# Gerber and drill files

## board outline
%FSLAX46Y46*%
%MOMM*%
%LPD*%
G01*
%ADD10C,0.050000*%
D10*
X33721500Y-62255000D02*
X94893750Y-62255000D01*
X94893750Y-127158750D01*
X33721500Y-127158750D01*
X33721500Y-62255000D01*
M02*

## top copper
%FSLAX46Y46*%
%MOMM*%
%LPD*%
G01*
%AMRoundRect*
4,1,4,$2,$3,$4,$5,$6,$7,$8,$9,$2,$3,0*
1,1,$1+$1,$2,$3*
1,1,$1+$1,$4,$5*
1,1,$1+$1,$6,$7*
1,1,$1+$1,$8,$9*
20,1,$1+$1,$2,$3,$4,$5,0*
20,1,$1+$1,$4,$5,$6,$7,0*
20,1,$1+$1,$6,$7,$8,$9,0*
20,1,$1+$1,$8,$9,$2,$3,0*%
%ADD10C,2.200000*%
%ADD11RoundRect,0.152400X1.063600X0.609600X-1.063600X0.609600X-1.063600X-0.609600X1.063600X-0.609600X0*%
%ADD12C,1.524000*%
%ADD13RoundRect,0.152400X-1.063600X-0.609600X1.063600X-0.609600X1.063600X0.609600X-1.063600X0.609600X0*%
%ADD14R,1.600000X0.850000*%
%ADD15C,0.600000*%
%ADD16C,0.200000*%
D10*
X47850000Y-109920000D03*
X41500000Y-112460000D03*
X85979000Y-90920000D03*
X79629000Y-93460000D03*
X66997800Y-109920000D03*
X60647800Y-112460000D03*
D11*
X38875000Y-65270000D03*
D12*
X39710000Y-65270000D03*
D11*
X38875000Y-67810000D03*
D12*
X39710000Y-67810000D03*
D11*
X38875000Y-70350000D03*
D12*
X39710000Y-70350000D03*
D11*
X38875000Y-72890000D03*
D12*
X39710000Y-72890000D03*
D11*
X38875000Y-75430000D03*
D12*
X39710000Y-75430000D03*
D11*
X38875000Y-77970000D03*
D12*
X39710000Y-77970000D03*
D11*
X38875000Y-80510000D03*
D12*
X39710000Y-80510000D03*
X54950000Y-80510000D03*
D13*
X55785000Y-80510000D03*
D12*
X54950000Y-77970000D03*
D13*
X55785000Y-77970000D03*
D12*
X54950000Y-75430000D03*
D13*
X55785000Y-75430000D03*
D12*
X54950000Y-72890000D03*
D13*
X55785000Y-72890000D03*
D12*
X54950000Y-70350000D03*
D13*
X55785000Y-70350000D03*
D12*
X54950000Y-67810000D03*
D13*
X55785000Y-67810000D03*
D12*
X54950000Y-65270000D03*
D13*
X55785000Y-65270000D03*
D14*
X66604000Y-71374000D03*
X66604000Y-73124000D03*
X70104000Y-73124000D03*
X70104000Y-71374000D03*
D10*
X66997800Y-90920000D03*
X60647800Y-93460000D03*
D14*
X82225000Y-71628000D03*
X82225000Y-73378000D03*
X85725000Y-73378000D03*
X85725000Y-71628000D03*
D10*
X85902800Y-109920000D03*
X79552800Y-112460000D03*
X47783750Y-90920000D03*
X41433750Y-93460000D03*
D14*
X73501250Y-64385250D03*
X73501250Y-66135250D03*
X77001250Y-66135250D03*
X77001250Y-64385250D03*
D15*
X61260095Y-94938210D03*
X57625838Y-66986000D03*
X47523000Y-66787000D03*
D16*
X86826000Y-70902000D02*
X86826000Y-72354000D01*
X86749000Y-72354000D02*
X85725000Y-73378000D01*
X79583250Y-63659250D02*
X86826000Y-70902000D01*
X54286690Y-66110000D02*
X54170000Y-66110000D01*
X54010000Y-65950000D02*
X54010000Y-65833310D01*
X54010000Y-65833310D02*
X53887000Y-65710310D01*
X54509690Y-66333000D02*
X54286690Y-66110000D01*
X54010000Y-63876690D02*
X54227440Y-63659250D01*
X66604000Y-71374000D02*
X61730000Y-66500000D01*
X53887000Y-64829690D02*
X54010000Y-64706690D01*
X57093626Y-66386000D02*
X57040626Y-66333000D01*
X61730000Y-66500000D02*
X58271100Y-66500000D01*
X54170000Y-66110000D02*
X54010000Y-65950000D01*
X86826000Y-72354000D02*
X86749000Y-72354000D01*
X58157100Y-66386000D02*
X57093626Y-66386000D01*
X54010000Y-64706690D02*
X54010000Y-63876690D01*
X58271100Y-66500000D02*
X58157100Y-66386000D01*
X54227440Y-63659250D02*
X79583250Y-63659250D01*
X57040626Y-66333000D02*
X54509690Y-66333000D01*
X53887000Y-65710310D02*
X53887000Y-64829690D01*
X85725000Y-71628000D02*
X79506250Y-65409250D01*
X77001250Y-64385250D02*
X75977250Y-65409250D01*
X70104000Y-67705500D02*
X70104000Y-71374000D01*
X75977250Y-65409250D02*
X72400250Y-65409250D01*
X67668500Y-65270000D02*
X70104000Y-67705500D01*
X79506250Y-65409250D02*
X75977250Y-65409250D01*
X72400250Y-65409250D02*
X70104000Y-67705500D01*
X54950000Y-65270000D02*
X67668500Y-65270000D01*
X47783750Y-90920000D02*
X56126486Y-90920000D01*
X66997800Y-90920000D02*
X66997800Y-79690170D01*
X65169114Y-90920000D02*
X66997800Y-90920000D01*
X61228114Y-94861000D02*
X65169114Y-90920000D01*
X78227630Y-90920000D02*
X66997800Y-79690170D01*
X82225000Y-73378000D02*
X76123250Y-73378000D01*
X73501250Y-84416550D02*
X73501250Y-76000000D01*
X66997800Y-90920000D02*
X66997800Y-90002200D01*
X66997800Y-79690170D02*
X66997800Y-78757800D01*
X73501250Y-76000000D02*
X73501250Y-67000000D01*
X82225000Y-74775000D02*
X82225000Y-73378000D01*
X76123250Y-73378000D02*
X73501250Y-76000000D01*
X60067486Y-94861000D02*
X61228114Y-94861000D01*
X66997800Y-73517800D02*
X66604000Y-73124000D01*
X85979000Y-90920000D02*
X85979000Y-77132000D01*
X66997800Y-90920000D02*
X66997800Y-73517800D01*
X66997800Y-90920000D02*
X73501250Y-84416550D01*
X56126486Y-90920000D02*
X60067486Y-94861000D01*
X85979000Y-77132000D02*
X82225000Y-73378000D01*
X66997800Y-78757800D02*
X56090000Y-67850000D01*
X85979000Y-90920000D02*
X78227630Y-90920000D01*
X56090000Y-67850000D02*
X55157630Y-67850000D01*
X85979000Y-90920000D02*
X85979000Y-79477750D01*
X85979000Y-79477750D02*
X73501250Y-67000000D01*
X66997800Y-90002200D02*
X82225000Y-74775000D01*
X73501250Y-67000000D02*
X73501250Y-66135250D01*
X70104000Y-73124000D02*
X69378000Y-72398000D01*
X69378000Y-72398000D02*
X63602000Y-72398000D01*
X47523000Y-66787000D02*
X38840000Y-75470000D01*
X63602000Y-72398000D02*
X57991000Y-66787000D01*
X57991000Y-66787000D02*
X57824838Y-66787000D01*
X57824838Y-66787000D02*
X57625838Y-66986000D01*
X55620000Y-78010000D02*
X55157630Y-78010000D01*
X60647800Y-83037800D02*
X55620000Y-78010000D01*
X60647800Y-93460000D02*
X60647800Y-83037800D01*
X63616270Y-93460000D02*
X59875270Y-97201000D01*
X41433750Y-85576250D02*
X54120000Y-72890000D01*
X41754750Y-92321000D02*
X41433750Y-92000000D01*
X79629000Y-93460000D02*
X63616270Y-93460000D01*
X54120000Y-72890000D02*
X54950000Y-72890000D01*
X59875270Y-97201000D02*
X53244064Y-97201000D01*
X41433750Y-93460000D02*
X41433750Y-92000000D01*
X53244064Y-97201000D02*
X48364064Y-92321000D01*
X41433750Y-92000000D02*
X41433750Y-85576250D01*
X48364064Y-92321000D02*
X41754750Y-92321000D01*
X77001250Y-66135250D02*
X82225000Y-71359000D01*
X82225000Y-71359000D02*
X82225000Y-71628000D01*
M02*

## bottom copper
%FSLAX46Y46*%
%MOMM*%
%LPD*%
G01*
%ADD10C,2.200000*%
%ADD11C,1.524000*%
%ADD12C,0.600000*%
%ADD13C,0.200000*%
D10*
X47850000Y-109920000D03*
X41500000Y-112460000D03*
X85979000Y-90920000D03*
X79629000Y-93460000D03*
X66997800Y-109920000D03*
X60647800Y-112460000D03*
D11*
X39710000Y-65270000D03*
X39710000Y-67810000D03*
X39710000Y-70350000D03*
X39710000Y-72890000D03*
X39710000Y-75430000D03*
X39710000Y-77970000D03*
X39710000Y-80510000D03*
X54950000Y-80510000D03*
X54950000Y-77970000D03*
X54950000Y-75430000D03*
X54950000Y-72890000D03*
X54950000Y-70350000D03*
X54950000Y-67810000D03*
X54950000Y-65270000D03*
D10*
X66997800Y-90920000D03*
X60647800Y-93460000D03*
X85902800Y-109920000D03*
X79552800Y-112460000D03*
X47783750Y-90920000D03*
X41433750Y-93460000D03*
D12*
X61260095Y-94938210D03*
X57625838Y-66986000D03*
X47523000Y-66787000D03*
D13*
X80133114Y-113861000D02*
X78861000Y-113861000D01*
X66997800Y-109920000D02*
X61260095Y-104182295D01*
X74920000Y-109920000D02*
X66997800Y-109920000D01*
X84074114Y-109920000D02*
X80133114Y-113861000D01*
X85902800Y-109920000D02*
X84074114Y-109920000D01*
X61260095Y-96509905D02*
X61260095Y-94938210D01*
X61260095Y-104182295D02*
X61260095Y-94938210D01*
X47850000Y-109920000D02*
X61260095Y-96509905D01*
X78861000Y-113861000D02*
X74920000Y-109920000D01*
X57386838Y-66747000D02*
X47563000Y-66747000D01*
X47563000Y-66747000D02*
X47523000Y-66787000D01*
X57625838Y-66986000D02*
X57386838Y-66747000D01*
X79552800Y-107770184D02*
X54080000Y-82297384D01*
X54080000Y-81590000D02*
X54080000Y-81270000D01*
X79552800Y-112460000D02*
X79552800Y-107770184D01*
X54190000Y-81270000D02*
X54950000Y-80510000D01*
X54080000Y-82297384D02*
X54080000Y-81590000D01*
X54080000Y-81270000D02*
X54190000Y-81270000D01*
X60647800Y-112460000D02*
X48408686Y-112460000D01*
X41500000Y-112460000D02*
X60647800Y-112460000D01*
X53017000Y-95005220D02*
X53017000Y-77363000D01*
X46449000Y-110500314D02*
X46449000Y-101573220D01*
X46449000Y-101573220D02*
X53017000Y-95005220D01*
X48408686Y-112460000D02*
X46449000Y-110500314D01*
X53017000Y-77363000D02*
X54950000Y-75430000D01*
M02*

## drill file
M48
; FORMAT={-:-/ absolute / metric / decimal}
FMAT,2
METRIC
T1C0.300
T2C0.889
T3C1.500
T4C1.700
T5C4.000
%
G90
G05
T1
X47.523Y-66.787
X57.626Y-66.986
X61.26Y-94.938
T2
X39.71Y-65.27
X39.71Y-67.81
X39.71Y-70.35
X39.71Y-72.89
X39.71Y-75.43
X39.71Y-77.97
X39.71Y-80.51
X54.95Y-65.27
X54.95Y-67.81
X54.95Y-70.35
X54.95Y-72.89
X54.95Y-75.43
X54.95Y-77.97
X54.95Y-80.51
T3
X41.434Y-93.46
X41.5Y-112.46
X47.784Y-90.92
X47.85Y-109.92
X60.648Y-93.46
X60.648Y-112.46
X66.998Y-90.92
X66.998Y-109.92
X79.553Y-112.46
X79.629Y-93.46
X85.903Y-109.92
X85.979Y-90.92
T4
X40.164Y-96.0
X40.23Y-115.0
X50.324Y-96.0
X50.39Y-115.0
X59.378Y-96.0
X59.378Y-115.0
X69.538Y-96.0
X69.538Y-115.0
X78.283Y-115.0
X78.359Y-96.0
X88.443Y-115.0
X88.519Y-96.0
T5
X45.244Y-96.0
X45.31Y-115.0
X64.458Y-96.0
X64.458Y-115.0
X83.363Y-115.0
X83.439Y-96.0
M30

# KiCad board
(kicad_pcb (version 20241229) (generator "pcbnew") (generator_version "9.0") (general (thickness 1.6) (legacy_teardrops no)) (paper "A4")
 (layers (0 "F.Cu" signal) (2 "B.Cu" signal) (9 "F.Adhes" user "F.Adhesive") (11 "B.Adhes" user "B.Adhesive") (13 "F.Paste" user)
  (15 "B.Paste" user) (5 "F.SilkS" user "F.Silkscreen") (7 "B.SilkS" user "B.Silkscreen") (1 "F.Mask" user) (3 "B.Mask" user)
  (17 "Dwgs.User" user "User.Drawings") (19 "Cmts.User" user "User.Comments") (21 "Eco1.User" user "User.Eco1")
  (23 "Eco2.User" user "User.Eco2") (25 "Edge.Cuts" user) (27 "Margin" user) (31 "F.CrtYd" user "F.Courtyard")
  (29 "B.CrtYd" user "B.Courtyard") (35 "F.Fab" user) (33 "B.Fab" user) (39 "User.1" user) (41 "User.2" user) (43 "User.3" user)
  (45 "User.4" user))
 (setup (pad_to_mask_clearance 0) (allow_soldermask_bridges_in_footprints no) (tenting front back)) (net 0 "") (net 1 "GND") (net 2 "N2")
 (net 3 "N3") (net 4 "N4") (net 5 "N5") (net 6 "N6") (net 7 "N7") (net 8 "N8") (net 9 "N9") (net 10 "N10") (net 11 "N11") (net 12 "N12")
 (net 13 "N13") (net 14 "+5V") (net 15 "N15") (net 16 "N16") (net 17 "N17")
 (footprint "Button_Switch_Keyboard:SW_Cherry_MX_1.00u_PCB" (layer "F.Cu") (at 47.85 109.92)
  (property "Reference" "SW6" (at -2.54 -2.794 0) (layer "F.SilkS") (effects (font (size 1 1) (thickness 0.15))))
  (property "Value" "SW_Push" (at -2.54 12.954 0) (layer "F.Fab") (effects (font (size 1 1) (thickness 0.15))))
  (pad "" np_thru_hole circle (at -7.62 5.08) (size 1.7 1.7) (drill 1.7) (layers "*.Cu" "*.Mask"))
  (pad "" np_thru_hole circle (at -2.54 5.08) (size 4 4) (drill 4) (layers "*.Cu" "*.Mask"))
  (pad "" np_thru_hole circle (at 2.54 5.08) (size 1.7 1.7) (drill 1.7) (layers "*.Cu" "*.Mask"))
  (pad "1" thru_hole circle (at 0 0) (size 2.2 2.2) (drill 1.5) (layers "*.Cu" "*.Mask") (remove_unused_layers no) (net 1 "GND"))
  (pad "2" thru_hole circle (at -6.35 2.54) (size 2.2 2.2) (drill 1.5) (layers "*.Cu" "*.Mask") (remove_unused_layers no) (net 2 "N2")))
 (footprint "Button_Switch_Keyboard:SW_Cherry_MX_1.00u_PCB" (layer "F.Cu") (at 85.979 90.92)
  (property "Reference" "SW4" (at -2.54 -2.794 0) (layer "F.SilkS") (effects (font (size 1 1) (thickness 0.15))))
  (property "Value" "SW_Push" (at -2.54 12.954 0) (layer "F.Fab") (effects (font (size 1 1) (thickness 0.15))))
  (pad "" np_thru_hole circle (at -7.62 5.08) (size 1.7 1.7) (drill 1.7) (layers "*.Cu" "*.Mask"))
  (pad "" np_thru_hole circle (at -2.54 5.08) (size 4 4) (drill 4) (layers "*.Cu" "*.Mask"))
  (pad "" np_thru_hole circle (at 2.54 5.08) (size 1.7 1.7) (drill 1.7) (layers "*.Cu" "*.Mask"))
  (pad "1" thru_hole circle (at 0 0) (size 2.2 2.2) (drill 1.5) (layers "*.Cu" "*.Mask") (remove_unused_layers no) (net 1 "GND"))
  (pad "2" thru_hole circle (at -6.35 2.54) (size 2.2 2.2) (drill 1.5) (layers "*.Cu" "*.Mask") (remove_unused_layers no) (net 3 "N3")))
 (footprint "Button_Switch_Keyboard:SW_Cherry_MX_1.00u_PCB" (layer "F.Cu") (at 66.9978 109.92)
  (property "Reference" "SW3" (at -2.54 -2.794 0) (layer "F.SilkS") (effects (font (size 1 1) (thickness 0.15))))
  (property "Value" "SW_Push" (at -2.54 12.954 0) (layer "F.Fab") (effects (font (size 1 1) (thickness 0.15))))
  (pad "" np_thru_hole circle (at -7.62 5.08) (size 1.7 1.7) (drill 1.7) (layers "*.Cu" "*.Mask"))
  (pad "" np_thru_hole circle (at -2.54 5.08) (size 4 4) (drill 4) (layers "*.Cu" "*.Mask"))
  (pad "" np_thru_hole circle (at 2.54 5.08) (size 1.7 1.7) (drill 1.7) (layers "*.Cu" "*.Mask"))
  (pad "1" thru_hole circle (at 0 0) (size 2.2 2.2) (drill 1.5) (layers "*.Cu" "*.Mask") (remove_unused_layers no) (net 1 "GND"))
  (pad "2" thru_hole circle (at -6.35 2.54) (size 2.2 2.2) (drill 1.5) (layers "*.Cu" "*.Mask") (remove_unused_layers no) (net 2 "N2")))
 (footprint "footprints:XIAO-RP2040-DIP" (layer "F.Cu") (at 47.33 72.89)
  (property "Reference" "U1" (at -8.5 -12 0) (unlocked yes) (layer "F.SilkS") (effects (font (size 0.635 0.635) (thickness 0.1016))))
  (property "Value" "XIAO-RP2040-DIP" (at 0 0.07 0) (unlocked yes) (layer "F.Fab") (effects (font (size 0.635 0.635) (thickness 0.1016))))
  (pad "1" smd roundrect (at -8.455 -7.62 180) (size 2.432 1.524) (layers "F.Cu" "F.Mask") (roundrect_rratio 0.1) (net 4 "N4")
   (thermal_bridge_angle 45))
  (pad "1" thru_hole circle (at -7.62 -7.62 180) (size 1.524 1.524) (drill 0.889) (layers "*.Cu" "*.Mask") (remove_unused_layers no)
   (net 4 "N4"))
  (pad "2" smd roundrect (at -8.455 -5.08 180) (size 2.432 1.524) (layers "F.Cu" "F.Mask") (roundrect_rratio 0.1) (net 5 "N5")
   (thermal_bridge_angle 45))
  (pad "2" thru_hole circle (at -7.62 -5.08 180) (size 1.524 1.524) (drill 0.889) (layers "*.Cu" "*.Mask") (remove_unused_layers no)
   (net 5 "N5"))
  (pad "3" smd roundrect (at -8.455 -2.54 180) (size 2.432 1.524) (layers "F.Cu" "F.Mask") (roundrect_rratio 0.1) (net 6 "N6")
   (thermal_bridge_angle 45))
  (pad "3" thru_hole circle (at -7.62 -2.54 180) (size 1.524 1.524) (drill 0.889) (layers "*.Cu" "*.Mask") (remove_unused_layers no)
   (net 6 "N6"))
  (pad "4" smd roundrect (at -8.455 0 180) (size 2.432 1.524) (layers "F.Cu" "F.Mask") (roundrect_rratio 0.1) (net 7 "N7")
   (thermal_bridge_angle 45))
  (pad "4" thru_hole circle (at -7.62 0 180) (size 1.524 1.524) (drill 0.889) (layers "*.Cu" "*.Mask") (remove_unused_layers no)
   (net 7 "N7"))
  (pad "5" smd roundrect (at -8.455 2.54 180) (size 2.432 1.524) (layers "F.Cu" "F.Mask") (roundrect_rratio 0.1) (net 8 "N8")
   (thermal_bridge_angle 45))
  (pad "5" thru_hole circle (at -7.62 2.54 180) (size 1.524 1.524) (drill 0.889) (layers "*.Cu" "*.Mask") (remove_unused_layers no)
   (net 8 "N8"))
  (pad "6" smd roundrect (at -8.455 5.08 180) (size 2.432 1.524) (layers "F.Cu" "F.Mask") (roundrect_rratio 0.1) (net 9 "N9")
   (thermal_bridge_angle 45))
  (pad "6" thru_hole circle (at -7.62 5.08 180) (size 1.524 1.524) (drill 0.889) (layers "*.Cu" "*.Mask") (remove_unused_layers no)
   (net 9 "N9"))
  (pad "7" smd roundrect (at -8.455 7.62 180) (size 2.432 1.524) (layers "F.Cu" "F.Mask") (roundrect_rratio 0.1) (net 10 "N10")
   (thermal_bridge_angle 45))
  (pad "7" thru_hole circle (at -7.62 7.62 180) (size 1.524 1.524) (drill 0.889) (layers "*.Cu" "*.Mask") (remove_unused_layers no)
   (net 10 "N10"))
  (pad "8" thru_hole circle (at 7.62 7.62) (size 1.524 1.524) (drill 0.889) (layers "*.Cu" "*.Mask") (remove_unused_layers no)
   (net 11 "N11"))
  (pad "8" smd roundrect (at 8.455 7.62) (size 2.432 1.524) (layers "F.Cu" "F.Mask") (roundrect_rratio 0.1) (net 11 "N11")
   (thermal_bridge_angle 45))
  (pad "9" thru_hole circle (at 7.62 5.08) (size 1.524 1.524) (drill 0.889) (layers "*.Cu" "*.Mask") (remove_unused_layers no)
   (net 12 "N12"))
  (pad "9" smd roundrect (at 8.455 5.08) (size 2.432 1.524) (layers "F.Cu" "F.Mask") (roundrect_rratio 0.1) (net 12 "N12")
   (thermal_bridge_angle 45))
  (pad "10" thru_hole circle (at 7.62 2.54) (size 1.524 1.524) (drill 0.889) (layers "*.Cu" "*.Mask") (remove_unused_layers no) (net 2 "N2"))
  (pad "10" smd roundrect (at 8.455 2.54) (size 2.432 1.524) (layers "F.Cu" "F.Mask") (roundrect_rratio 0.1) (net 2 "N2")
   (thermal_bridge_angle 45))
  (pad "11" thru_hole circle (at 7.62 0) (size 1.524 1.524) (drill 0.889) (layers "*.Cu" "*.Mask") (remove_unused_layers no) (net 3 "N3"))
  (pad "11" smd roundrect (at 8.455 0) (size 2.432 1.524) (layers "F.Cu" "F.Mask") (roundrect_rratio 0.1) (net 3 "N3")
   (thermal_bridge_angle 45))
  (pad "12" thru_hole circle (at 7.62 -2.54) (size 1.524 1.524) (drill 0.889) (layers "*.Cu" "*.Mask") (remove_unused_layers no)
   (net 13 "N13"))
  (pad "12" smd roundrect (at 8.455 -2.54) (size 2.432 1.524) (layers "F.Cu" "F.Mask") (roundrect_rratio 0.1) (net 13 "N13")
   (thermal_bridge_angle 45))
  (pad "13" thru_hole circle (at 7.62 -5.08) (size 1.524 1.524) (drill 0.889) (layers "*.Cu" "*.Mask") (remove_unused_layers no)
   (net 1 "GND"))
  (pad "13" smd roundrect (at 8.455 -5.08) (size 2.432 1.524) (layers "F.Cu" "F.Mask") (roundrect_rratio 0.1) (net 1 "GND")
   (thermal_bridge_angle 45))
  (pad "14" thru_hole circle (at 7.62 -7.62) (size 1.524 1.524) (drill 0.889) (layers "*.Cu" "*.Mask") (remove_unused_layers no)
   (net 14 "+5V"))
  (pad "14" smd roundrect (at 8.455 -7.62) (size 2.432 1.524) (layers "F.Cu" "F.Mask") (roundrect_rratio 0.1) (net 14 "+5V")
   (thermal_bridge_angle 45)))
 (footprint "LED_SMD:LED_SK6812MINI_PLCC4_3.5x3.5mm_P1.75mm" (layer "F.Cu") (at 68.354 72.249)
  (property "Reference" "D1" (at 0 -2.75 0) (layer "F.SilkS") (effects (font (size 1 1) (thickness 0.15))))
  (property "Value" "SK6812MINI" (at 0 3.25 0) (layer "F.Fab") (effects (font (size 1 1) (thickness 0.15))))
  (pad "1" smd rect (at -1.75 -0.875) (size 1.6 0.85) (layers "F.Cu" "F.Mask" "F.Paste") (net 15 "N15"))
  (pad "2" smd rect (at -1.75 0.875) (size 1.6 0.85) (layers "F.Cu" "F.Mask" "F.Paste") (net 1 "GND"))
  (pad "3" smd rect (at 1.75 0.875) (size 1.6 0.85) (layers "F.Cu" "F.Mask" "F.Paste") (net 8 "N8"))
  (pad "4" smd rect (at 1.75 -0.875) (size 1.6 0.85) (layers "F.Cu" "F.Mask" "F.Paste") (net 14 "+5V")))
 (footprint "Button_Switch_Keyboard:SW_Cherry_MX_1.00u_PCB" (layer "F.Cu") (at 66.9978 90.92)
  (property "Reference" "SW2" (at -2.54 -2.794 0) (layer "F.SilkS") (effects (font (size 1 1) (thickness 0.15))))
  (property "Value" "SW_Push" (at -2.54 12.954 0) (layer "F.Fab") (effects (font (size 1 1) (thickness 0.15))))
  (pad "" np_thru_hole circle (at -7.62 5.08) (size 1.7 1.7) (drill 1.7) (layers "*.Cu" "*.Mask"))
  (pad "" np_thru_hole circle (at -2.54 5.08) (size 4 4) (drill 4) (layers "*.Cu" "*.Mask"))
  (pad "" np_thru_hole circle (at 2.54 5.08) (size 1.7 1.7) (drill 1.7) (layers "*.Cu" "*.Mask"))
  (pad "1" thru_hole circle (at 0 0) (size 2.2 2.2) (drill 1.5) (layers "*.Cu" "*.Mask") (remove_unused_layers no) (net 1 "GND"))
  (pad "2" thru_hole circle (at -6.35 2.54) (size 2.2 2.2) (drill 1.5) (layers "*.Cu" "*.Mask") (remove_unused_layers no) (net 12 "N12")))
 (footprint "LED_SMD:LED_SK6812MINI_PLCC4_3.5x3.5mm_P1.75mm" (layer "F.Cu") (at 83.975 72.503)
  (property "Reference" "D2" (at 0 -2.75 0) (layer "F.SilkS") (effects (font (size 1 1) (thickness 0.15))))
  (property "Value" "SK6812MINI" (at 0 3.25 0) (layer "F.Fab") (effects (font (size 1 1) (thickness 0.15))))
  (pad "1" smd rect (at -1.75 -0.875) (size 1.6 0.85) (layers "F.Cu" "F.Mask" "F.Paste") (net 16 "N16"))
  (pad "2" smd rect (at -1.75 0.875) (size 1.6 0.85) (layers "F.Cu" "F.Mask" "F.Paste") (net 1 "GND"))
  (pad "3" smd rect (at 1.75 0.875) (size 1.6 0.85) (layers "F.Cu" "F.Mask" "F.Paste") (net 15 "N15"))
  (pad "4" smd rect (at 1.75 -0.875) (size 1.6 0.85) (layers "F.Cu" "F.Mask" "F.Paste") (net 14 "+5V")))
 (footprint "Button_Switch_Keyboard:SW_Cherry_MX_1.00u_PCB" (layer "F.Cu") (at 85.9028 109.92)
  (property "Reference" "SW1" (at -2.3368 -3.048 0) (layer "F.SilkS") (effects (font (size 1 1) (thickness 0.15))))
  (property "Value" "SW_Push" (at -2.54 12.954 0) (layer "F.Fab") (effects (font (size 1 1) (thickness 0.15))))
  (pad "" np_thru_hole circle (at -7.62 5.08) (size 1.7 1.7) (drill 1.7) (layers "*.Cu" "*.Mask"))
  (pad "" np_thru_hole circle (at -2.54 5.08) (size 4 4) (drill 4) (layers "*.Cu" "*.Mask"))
  (pad "" np_thru_hole circle (at 2.54 5.08) (size 1.7 1.7) (drill 1.7) (layers "*.Cu" "*.Mask"))
  (pad "1" thru_hole circle (at 0 0) (size 2.2 2.2) (drill 1.5) (layers "*.Cu" "*.Mask") (remove_unused_layers no) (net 1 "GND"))
  (pad "2" thru_hole circle (at -6.35 2.54) (size 2.2 2.2) (drill 1.5) (layers "*.Cu" "*.Mask") (remove_unused_layers no) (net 11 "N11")))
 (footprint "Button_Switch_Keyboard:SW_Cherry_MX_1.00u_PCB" (layer "F.Cu") (at 47.78375 90.92)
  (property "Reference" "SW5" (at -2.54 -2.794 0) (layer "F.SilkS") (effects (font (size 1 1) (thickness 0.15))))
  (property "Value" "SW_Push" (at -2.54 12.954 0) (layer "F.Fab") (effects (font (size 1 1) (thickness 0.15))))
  (pad "" np_thru_hole circle (at -7.62 5.08) (size 1.7 1.7) (drill 1.7) (layers "*.Cu" "*.Mask"))
  (pad "" np_thru_hole circle (at -2.54 5.08) (size 4 4) (drill 4) (layers "*.Cu" "*.Mask"))
  (pad "" np_thru_hole circle (at 2.54 5.08) (size 1.7 1.7) (drill 1.7) (layers "*.Cu" "*.Mask"))
  (pad "1" thru_hole circle (at 0 0) (size 2.2 2.2) (drill 1.5) (layers "*.Cu" "*.Mask") (remove_unused_layers no) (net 1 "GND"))
  (pad "2" thru_hole circle (at -6.35 2.54) (size 2.2 2.2) (drill 1.5) (layers "*.Cu" "*.Mask") (remove_unused_layers no) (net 3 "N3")))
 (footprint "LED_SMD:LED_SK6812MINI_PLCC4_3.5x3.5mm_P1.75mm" (layer "F.Cu") (at 75.25125 65.26025)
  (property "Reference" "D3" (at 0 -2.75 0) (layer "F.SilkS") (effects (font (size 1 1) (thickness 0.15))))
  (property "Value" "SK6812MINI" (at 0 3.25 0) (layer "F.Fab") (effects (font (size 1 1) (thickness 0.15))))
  (pad "1" smd rect (at -1.75 -0.875) (size 1.6 0.85) (layers "F.Cu" "F.Mask" "F.Paste") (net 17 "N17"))
  (pad "2" smd rect (at -1.75 0.875) (size 1.6 0.85) (layers "F.Cu" "F.Mask" "F.Paste") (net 1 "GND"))
  (pad "3" smd rect (at 1.75 0.875) (size 1.6 0.85) (layers "F.Cu" "F.Mask" "F.Paste") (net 16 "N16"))
  (pad "4" smd rect (at 1.75 -0.875) (size 1.6 0.85) (layers "F.Cu" "F.Mask" "F.Paste") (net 14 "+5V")))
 (gr_rect (start 33.7215 62.255) (end 94.89375 127.15875) (stroke (width 0.05) (type default)) (fill no) (layer "Edge.Cuts"))
 (segment (start 86.826 70.902) (end 86.826 72.354) (width 0.2) (layer "F.Cu") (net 15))
 (segment (start 86.749 72.354) (end 85.725 73.378) (width 0.2) (layer "F.Cu") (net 15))
 (segment (start 79.58325 63.65925) (end 86.826 70.902) (width 0.2) (layer "F.Cu") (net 15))
 (segment (start 54.28669 66.11) (end 54.17 66.11) (width 0.2) (layer "F.Cu") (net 15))
 (segment (start 54.01 65.95) (end 54.01 65.83331) (width 0.2) (layer "F.Cu") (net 15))
 (segment (start 54.01 65.83331) (end 53.887 65.71031) (width 0.2) (layer "F.Cu") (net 15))
 (segment (start 54.50969 66.333) (end 54.28669 66.11) (width 0.2) (layer "F.Cu") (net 15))
 (segment (start 54.01 63.87669) (end 54.22744 63.65925) (width 0.2) (layer "F.Cu") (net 15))
 (segment (start 66.604 71.374) (end 61.73 66.5) (width 0.2) (layer "F.Cu") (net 15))
 (segment (start 53.887 64.82969) (end 54.01 64.70669) (width 0.2) (layer "F.Cu") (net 15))
 (segment (start 57.093626 66.386) (end 57.040626 66.333) (width 0.2) (layer "F.Cu") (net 15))
 (segment (start 61.73 66.5) (end 58.2711 66.5) (width 0.2) (layer "F.Cu") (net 15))
 (segment (start 54.17 66.11) (end 54.01 65.95) (width 0.2) (layer "F.Cu") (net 15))
 (segment (start 86.826 72.354) (end 86.749 72.354) (width 0.2) (layer "F.Cu") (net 15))
 (segment (start 58.1571 66.386) (end 57.093626 66.386) (width 0.2) (layer "F.Cu") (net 15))
 (segment (start 54.01 64.70669) (end 54.01 63.87669) (width 0.2) (layer "F.Cu") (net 15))
 (segment (start 58.2711 66.5) (end 58.1571 66.386) (width 0.2) (layer "F.Cu") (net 15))
 (segment (start 54.22744 63.65925) (end 79.58325 63.65925) (width 0.2) (layer "F.Cu") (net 15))
 (segment (start 57.040626 66.333) (end 54.50969 66.333) (width 0.2) (layer "F.Cu") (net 15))
 (segment (start 53.887 65.71031) (end 53.887 64.82969) (width 0.2) (layer "F.Cu") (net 15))
 (segment (start 85.725 71.628) (end 79.50625 65.40925) (width 0.2) (layer "F.Cu") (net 14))
 (segment (start 77.00125 64.38525) (end 75.97725 65.40925) (width 0.2) (layer "F.Cu") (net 14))
 (segment (start 70.104 67.7055) (end 70.104 71.374) (width 0.2) (layer "F.Cu") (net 14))
 (segment (start 75.97725 65.40925) (end 72.40025 65.40925) (width 0.2) (layer "F.Cu") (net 14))
 (segment (start 67.6685 65.27) (end 70.104 67.7055) (width 0.2) (layer "F.Cu") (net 14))
 (segment (start 79.50625 65.40925) (end 75.97725 65.40925) (width 0.2) (layer "F.Cu") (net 14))
 (segment (start 72.40025 65.40925) (end 70.104 67.7055) (width 0.2) (layer "F.Cu") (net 14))
 (segment (start 54.95 65.27) (end 67.6685 65.27) (width 0.2) (layer "F.Cu") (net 14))
 (segment (start 47.78375 90.92) (end 56.126486 90.92) (width 0.2) (layer "F.Cu") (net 1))
 (segment (start 66.9978 90.92) (end 66.9978 79.69017) (width 0.2) (layer "F.Cu") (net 1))
 (segment (start 65.169114 90.92) (end 66.9978 90.92) (width 0.2) (layer "F.Cu") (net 1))
 (segment (start 61.228114 94.861) (end 65.169114 90.92) (width 0.2) (layer "F.Cu") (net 1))
 (segment (start 78.22763 90.92) (end 66.9978 79.69017) (width 0.2) (layer "F.Cu") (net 1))
 (segment (start 82.225 73.378) (end 76.12325 73.378) (width 0.2) (layer "F.Cu") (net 1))
 (segment (start 73.50125 84.41655) (end 73.50125 76) (width 0.2) (layer "F.Cu") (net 1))
 (segment (start 66.9978 90.92) (end 66.9978 90.0022) (width 0.2) (layer "F.Cu") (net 1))
 (segment (start 66.9978 79.69017) (end 66.9978 78.7578) (width 0.2) (layer "F.Cu") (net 1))
 (segment (start 73.50125 76) (end 73.50125 67) (width 0.2) (layer "F.Cu") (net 1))
 (segment (start 82.225 74.775) (end 82.225 73.378) (width 0.2) (layer "F.Cu") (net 1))
 (segment (start 76.12325 73.378) (end 73.50125 76) (width 0.2) (layer "F.Cu") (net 1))
 (segment (start 60.067486 94.861) (end 61.228114 94.861) (width 0.2) (layer "F.Cu") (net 1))
 (segment (start 66.9978 73.5178) (end 66.604 73.124) (width 0.2) (layer "F.Cu") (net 1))
 (segment (start 85.979 90.92) (end 85.979 77.132) (width 0.2) (layer "F.Cu") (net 1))
 (segment (start 66.9978 90.92) (end 66.9978 73.5178) (width 0.2) (layer "F.Cu") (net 1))
 (segment (start 66.9978 90.92) (end 73.50125 84.41655) (width 0.2) (layer "F.Cu") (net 1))
 (segment (start 56.126486 90.92) (end 60.067486 94.861) (width 0.2) (layer "F.Cu") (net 1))
 (segment (start 85.979 77.132) (end 82.225 73.378) (width 0.2) (layer "F.Cu") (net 1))
 (segment (start 66.9978 78.7578) (end 56.09 67.85) (width 0.2) (layer "F.Cu") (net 1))
 (segment (start 85.979 90.92) (end 78.22763 90.92) (width 0.2) (layer "F.Cu") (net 1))
 (segment (start 56.09 67.85) (end 55.15763 67.85) (width 0.2) (layer "F.Cu") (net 1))
 (segment (start 85.979 90.92) (end 85.979 79.47775) (width 0.2) (layer "F.Cu") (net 1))
 (segment (start 85.979 79.47775) (end 73.50125 67) (width 0.2) (layer "F.Cu") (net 1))
 (segment (start 66.9978 90.0022) (end 82.225 74.775) (width 0.2) (layer "F.Cu") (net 1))
 (segment (start 73.50125 67) (end 73.50125 66.13525) (width 0.2) (layer "F.Cu") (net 1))
 (via (at 61.260095 94.93821) (size 0.6) (drill 0.3) (layers "F.Cu" "B.Cu") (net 1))
 (segment (start 80.133114 113.861) (end 78.861 113.861) (width 0.2) (layer "B.Cu") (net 1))
 (segment (start 66.9978 109.92) (end 61.260095 104.182295) (width 0.2) (layer "B.Cu") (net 1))
 (segment (start 74.92 109.92) (end 66.9978 109.92) (width 0.2) (layer "B.Cu") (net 1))
 (segment (start 84.074114 109.92) (end 80.133114 113.861) (width 0.2) (layer "B.Cu") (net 1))
 (segment (start 85.9028 109.92) (end 84.074114 109.92) (width 0.2) (layer "B.Cu") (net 1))
 (segment (start 61.260095 96.509905) (end 61.260095 94.93821) (width 0.2) (layer "B.Cu") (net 1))
 (segment (start 61.260095 104.182295) (end 61.260095 94.93821) (width 0.2) (layer "B.Cu") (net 1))
 (segment (start 47.85 109.92) (end 61.260095 96.509905) (width 0.2) (layer "B.Cu") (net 1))
 (segment (start 78.861 113.861) (end 74.92 109.92) (width 0.2) (layer "B.Cu") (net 1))
 (segment (start 70.104 73.124) (end 69.378 72.398) (width 0.2) (layer "F.Cu") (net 8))
 (segment (start 69.378 72.398) (end 63.602 72.398) (width 0.2) (layer "F.Cu") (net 8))
 (segment (start 47.523 66.787) (end 38.84 75.47) (width 0.2) (layer "F.Cu") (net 8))
 (segment (start 63.602 72.398) (end 57.991 66.787) (width 0.2) (layer "F.Cu") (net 8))
 (segment (start 57.991 66.787) (end 57.824838 66.787) (width 0.2) (layer "F.Cu") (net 8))
 (segment (start 57.824838 66.787) (end 57.625838 66.986) (width 0.2) (layer "F.Cu") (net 8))
 (via (at 57.625838 66.986) (size 0.6) (drill 0.3) (layers "F.Cu" "B.Cu") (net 8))
 (via (at 47.523 66.787) (size 0.6) (drill 0.3) (layers "F.Cu" "B.Cu") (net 8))
 (segment (start 57.386838 66.747) (end 47.563 66.747) (width 0.2) (layer "B.Cu") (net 8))
 (segment (start 47.563 66.747) (end 47.523 66.787) (width 0.2) (layer "B.Cu") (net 8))
 (segment (start 57.625838 66.986) (end 57.386838 66.747) (width 0.2) (layer "B.Cu") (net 8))
 (segment (start 79.5528 107.770184) (end 54.08 82.297384) (width 0.2) (layer "B.Cu") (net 11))
 (segment (start 54.08 81.59) (end 54.08 81.27) (width 0.2) (layer "B.Cu") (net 11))
 (segment (start 79.5528 112.46) (end 79.5528 107.770184) (width 0.2) (layer "B.Cu") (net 11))
 (segment (start 54.19 81.27) (end 54.95 80.51) (width 0.2) (layer "B.Cu") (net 11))
 (segment (start 54.08 82.297384) (end 54.08 81.59) (width 0.2) (layer "B.Cu") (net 11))
 (segment (start 54.08 81.27) (end 54.19 81.27) (width 0.2) (layer "B.Cu") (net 11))
 (segment (start 55.62 78.01) (end 55.15763 78.01) (width 0.2) (layer "F.Cu") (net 12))
 (segment (start 60.6478 83.0378) (end 55.62 78.01) (width 0.2) (layer "F.Cu") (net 12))
 (segment (start 60.6478 93.46) (end 60.6478 83.0378) (width 0.2) (layer "F.Cu") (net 12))
 (segment (start 60.6478 112.46) (end 48.408686 112.46) (width 0.2) (layer "B.Cu") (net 2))
 (segment (start 41.5 112.46) (end 60.6478 112.46) (width 0.2) (layer "B.Cu") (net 2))
 (segment (start 53.017 95.00522) (end 53.017 77.363) (width 0.2) (layer "B.Cu") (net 2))
 (segment (start 46.449 110.500314) (end 46.449 101.57322) (width 0.2) (layer "B.Cu") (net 2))
 (segment (start 46.449 101.57322) (end 53.017 95.00522) (width 0.2) (layer "B.Cu") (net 2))
 (segment (start 48.408686 112.46) (end 46.449 110.500314) (width 0.2) (layer "B.Cu") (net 2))
 (segment (start 53.017 77.363) (end 54.95 75.43) (width 0.2) (layer "B.Cu") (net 2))
 (segment (start 63.61627 93.46) (end 59.87527 97.201) (width 0.2) (layer "F.Cu") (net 3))
 (segment (start 41.43375 85.57625) (end 54.12 72.89) (width 0.2) (layer "F.Cu") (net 3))
 (segment (start 41.75475 92.321) (end 41.43375 92) (width 0.2) (layer "F.Cu") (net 3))
 (segment (start 79.629 93.46) (end 63.61627 93.46) (width 0.2) (layer "F.Cu") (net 3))
 (segment (start 54.12 72.89) (end 54.95 72.89) (width 0.2) (layer "F.Cu") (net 3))
 (segment (start 59.87527 97.201) (end 53.244064 97.201) (width 0.2) (layer "F.Cu") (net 3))
 (segment (start 41.43375 93.46) (end 41.43375 92) (width 0.2) (layer "F.Cu") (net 3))
 (segment (start 53.244064 97.201) (end 48.364064 92.321) (width 0.2) (layer "F.Cu") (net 3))
 (segment (start 41.43375 92) (end 41.43375 85.57625) (width 0.2) (layer "F.Cu") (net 3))
 (segment (start 48.364064 92.321) (end 41.75475 92.321) (width 0.2) (layer "F.Cu") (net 3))
 (segment (start 77.00125 66.13525) (end 82.225 71.359) (width 0.2) (layer "F.Cu") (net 16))
 (segment (start 82.225 71.359) (end 82.225 71.628) (width 0.2) (layer "F.Cu") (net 16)))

